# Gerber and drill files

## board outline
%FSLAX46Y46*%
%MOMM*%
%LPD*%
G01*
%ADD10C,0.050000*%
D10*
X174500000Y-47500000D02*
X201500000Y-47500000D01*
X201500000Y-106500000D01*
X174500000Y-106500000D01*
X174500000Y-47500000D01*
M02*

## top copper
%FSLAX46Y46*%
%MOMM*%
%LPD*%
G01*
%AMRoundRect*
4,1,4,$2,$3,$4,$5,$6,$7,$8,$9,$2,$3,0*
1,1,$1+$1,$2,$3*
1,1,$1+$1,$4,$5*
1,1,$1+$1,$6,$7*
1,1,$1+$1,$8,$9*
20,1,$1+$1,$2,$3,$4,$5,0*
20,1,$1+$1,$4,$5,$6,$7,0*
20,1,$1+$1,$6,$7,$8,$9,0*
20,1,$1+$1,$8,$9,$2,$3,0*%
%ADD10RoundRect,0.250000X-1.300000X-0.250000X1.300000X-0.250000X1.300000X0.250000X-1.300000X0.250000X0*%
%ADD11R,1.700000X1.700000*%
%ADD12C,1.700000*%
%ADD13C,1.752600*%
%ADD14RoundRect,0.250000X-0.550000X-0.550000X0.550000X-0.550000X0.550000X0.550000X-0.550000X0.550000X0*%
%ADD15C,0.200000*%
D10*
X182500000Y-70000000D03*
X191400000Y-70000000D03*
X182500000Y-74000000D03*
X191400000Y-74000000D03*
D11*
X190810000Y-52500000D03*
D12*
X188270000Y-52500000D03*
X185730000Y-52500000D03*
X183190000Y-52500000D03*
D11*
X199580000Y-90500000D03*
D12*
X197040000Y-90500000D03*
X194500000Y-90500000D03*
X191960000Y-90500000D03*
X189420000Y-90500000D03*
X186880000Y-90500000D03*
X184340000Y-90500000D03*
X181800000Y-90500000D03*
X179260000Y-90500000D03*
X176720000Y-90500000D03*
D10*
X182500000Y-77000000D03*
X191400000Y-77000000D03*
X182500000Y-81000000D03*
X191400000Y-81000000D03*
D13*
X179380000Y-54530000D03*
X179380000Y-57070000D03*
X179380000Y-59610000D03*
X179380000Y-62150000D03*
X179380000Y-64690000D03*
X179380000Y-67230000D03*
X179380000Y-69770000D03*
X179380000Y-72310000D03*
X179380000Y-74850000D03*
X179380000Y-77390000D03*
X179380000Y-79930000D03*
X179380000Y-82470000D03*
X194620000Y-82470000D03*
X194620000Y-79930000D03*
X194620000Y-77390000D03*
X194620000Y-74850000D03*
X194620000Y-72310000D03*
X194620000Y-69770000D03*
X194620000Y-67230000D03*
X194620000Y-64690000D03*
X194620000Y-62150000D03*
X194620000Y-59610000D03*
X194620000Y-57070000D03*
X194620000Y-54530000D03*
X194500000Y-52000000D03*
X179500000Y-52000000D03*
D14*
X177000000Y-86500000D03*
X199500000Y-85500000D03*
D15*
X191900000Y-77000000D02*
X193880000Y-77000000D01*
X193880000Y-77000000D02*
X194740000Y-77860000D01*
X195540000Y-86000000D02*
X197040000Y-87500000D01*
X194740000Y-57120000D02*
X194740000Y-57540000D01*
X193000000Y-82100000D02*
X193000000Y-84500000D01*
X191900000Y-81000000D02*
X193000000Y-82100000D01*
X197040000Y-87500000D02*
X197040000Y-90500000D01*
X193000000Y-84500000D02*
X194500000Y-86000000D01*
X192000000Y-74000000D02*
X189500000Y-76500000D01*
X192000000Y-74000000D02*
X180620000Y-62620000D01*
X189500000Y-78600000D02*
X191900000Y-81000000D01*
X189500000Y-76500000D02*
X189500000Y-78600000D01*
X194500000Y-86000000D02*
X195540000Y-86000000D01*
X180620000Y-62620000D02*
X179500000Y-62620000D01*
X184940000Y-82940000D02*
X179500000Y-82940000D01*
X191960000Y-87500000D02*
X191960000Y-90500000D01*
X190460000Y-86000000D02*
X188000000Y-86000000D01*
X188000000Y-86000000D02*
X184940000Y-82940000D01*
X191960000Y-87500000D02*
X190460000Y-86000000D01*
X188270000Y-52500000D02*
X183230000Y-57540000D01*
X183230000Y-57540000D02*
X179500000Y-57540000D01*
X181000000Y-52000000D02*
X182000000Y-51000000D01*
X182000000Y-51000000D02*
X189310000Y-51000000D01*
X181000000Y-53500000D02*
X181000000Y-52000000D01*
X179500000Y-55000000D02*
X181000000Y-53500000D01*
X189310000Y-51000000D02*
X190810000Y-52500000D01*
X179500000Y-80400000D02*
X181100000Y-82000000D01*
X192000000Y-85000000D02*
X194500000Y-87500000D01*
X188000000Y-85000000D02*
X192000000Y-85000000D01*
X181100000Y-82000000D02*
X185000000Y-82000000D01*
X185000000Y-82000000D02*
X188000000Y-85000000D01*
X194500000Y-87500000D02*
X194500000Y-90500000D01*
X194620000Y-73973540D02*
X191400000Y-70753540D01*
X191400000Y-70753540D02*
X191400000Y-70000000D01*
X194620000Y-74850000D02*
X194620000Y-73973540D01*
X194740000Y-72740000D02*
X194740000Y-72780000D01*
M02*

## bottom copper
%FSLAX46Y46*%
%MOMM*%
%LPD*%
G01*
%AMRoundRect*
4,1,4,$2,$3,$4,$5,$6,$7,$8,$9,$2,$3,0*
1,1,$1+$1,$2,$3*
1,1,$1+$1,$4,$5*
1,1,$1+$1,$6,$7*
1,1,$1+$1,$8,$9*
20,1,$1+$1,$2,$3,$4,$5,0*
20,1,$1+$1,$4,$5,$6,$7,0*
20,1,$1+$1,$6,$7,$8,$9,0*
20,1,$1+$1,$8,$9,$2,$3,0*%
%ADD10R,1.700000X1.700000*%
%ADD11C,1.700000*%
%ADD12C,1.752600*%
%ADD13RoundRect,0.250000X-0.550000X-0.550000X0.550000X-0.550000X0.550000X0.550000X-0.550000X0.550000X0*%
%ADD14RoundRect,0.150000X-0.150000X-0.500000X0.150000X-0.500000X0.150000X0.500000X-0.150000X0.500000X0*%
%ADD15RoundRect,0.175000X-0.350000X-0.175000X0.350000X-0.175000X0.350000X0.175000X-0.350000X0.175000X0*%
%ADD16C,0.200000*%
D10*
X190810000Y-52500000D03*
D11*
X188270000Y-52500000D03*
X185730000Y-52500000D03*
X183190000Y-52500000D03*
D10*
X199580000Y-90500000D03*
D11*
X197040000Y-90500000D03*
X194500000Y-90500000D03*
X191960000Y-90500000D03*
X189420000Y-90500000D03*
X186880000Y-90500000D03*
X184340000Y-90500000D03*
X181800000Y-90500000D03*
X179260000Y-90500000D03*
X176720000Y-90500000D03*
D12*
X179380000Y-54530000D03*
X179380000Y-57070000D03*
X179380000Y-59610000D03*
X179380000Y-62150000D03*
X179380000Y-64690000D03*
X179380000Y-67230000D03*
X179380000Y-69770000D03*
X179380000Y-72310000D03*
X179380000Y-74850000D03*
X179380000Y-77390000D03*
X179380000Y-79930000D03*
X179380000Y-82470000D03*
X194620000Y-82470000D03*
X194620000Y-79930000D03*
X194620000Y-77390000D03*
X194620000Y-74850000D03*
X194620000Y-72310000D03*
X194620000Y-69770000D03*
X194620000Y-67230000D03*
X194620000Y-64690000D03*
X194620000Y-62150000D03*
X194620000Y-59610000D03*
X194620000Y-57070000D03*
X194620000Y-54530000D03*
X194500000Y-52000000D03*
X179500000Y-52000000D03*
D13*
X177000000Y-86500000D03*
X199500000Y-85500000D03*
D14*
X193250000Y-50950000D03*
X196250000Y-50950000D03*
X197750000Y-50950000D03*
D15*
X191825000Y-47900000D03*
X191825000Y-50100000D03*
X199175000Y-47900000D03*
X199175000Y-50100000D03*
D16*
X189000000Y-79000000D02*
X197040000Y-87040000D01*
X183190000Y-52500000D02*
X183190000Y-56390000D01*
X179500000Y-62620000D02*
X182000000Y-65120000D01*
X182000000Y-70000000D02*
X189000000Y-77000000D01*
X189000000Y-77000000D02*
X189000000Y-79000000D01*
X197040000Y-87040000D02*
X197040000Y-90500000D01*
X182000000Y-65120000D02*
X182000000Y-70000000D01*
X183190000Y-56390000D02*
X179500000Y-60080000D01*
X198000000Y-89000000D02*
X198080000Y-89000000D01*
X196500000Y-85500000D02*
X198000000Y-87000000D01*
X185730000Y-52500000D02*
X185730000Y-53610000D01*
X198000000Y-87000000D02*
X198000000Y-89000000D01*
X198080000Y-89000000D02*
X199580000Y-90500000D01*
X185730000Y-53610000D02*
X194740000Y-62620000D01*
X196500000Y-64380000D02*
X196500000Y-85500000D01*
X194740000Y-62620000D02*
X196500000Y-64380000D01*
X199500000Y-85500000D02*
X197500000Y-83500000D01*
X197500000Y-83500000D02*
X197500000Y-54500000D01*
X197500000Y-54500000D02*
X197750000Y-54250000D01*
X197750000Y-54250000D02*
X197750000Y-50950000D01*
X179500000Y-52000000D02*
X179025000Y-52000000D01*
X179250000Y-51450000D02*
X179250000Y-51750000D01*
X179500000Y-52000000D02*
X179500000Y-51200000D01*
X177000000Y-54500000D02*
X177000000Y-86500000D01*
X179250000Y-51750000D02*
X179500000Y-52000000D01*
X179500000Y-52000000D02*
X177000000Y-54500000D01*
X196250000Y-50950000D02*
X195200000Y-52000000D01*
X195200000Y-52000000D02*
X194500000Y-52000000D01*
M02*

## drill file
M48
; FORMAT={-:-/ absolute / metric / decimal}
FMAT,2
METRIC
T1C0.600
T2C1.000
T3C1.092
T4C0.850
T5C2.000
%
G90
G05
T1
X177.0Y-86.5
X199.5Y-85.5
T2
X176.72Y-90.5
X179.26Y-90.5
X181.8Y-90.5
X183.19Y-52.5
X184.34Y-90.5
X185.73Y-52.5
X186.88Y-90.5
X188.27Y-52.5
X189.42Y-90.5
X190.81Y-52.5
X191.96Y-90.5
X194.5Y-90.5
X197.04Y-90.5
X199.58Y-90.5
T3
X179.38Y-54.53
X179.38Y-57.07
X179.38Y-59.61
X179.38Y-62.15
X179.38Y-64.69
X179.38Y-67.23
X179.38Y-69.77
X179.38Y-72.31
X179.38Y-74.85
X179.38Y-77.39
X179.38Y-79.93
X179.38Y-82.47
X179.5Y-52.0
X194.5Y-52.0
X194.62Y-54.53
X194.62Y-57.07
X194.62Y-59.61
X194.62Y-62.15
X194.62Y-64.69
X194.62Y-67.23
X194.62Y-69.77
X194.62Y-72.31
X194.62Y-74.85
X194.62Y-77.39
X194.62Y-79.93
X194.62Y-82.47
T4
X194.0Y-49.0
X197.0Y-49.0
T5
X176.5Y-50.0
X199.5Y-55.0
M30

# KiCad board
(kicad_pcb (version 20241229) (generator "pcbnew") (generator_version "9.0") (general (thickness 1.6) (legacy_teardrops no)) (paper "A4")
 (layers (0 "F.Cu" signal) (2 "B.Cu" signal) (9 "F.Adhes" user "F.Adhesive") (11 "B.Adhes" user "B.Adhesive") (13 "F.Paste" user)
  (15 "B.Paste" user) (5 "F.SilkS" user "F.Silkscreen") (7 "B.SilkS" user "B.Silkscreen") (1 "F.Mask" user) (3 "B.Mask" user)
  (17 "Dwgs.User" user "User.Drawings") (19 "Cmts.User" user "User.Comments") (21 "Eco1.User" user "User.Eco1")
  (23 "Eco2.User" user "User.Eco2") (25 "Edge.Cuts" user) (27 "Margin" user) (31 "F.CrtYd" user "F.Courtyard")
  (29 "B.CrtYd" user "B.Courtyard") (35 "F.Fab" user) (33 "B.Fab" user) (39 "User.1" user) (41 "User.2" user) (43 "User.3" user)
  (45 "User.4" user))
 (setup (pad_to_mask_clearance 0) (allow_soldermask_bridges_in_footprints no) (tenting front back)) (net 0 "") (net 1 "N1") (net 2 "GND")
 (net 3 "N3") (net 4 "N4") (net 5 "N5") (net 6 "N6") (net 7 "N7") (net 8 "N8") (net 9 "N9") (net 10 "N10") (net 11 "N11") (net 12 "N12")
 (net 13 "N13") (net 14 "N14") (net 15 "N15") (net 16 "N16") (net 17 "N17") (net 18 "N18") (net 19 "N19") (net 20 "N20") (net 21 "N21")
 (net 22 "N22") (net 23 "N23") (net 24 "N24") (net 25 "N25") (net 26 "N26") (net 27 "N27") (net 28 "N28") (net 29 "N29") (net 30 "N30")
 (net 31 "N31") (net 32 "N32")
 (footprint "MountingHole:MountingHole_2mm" (layer "F.Cu") (at 176.5 50)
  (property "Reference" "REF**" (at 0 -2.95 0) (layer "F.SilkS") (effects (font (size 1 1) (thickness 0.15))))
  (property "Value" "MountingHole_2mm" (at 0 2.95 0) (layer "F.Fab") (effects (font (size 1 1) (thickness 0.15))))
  (pad "" np_thru_hole circle (at 0 0) (size 2 2) (drill 2) (layers "*.Cu" "*.Mask")))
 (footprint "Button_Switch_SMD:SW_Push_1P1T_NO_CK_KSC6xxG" (layer "F.Cu") (at 186.95 72)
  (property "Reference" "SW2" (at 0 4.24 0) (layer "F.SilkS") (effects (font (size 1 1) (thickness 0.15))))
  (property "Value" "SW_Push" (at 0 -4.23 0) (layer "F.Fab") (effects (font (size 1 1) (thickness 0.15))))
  (pad "1" smd roundrect (at -4.45 -2) (size 3.1 1) (layers "F.Cu" "F.Mask" "F.Paste") (roundrect_rratio 0.25) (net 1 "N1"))
  (pad "1" smd roundrect (at 4.45 -2) (size 3.1 1) (layers "F.Cu" "F.Mask" "F.Paste") (roundrect_rratio 0.25) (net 1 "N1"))
  (pad "2" smd roundrect (at -4.45 2) (size 3.1 1) (layers "F.Cu" "F.Mask" "F.Paste") (roundrect_rratio 0.25) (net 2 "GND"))
  (pad "2" smd roundrect (at 4.45 2) (size 3.1 1) (layers "F.Cu" "F.Mask" "F.Paste") (roundrect_rratio 0.25) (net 2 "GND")))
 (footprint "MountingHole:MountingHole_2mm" (layer "F.Cu") (at 199.5 55)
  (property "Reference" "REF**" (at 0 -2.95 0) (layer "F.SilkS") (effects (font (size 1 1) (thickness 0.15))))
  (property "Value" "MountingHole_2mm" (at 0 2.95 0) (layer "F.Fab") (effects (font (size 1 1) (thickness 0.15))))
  (pad "" np_thru_hole circle (at 0 0) (size 2 2) (drill 2) (layers "*.Cu" "*.Mask")))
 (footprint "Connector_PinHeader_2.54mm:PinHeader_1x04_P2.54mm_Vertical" (layer "F.Cu") (at 190.81 52.5 -90)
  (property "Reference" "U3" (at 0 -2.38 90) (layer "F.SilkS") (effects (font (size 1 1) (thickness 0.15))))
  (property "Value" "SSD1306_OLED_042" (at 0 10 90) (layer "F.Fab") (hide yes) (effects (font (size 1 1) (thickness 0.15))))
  (pad "1" thru_hole rect (at 0 0 270) (size 1.7 1.7) (drill 1) (layers "*.Cu" "*.Mask") (remove_unused_layers no) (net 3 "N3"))
  (pad "2" thru_hole circle (at 0 2.54 270) (size 1.7 1.7) (drill 1) (layers "*.Cu" "*.Mask") (remove_unused_layers no) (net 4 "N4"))
  (pad "3" thru_hole circle (at 0 5.08 270) (size 1.7 1.7) (drill 1) (layers "*.Cu" "*.Mask") (remove_unused_layers no) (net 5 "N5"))
  (pad "4" thru_hole circle (at 0 7.62 270) (size 1.7 1.7) (drill 1) (layers "*.Cu" "*.Mask") (remove_unused_layers no) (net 2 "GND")))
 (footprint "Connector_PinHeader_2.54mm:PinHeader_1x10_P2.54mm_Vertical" (layer "F.Cu") (at 199.58 90.5 -90)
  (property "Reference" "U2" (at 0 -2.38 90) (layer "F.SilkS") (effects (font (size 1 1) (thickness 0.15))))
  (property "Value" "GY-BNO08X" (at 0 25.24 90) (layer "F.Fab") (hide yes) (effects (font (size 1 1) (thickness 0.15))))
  (pad "1" thru_hole rect (at 0 0 270) (size 1.7 1.7) (drill 1) (layers "*.Cu" "*.Mask") (remove_unused_layers no) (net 5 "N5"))
  (pad "2" thru_hole circle (at 0 2.54 270) (size 1.7 1.7) (drill 1) (layers "*.Cu" "*.Mask") (remove_unused_layers no) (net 2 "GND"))
  (pad "3" thru_hole circle (at 0 5.08 270) (size 1.7 1.7) (drill 1) (layers "*.Cu" "*.Mask") (remove_unused_layers no) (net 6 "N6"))
  (pad "4" thru_hole circle (at 0 7.62 270) (size 1.7 1.7) (drill 1) (layers "*.Cu" "*.Mask") (remove_unused_layers no) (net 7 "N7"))
  (pad "5" thru_hole circle (at 0 10.16 270) (size 1.7 1.7) (drill 1) (layers "*.Cu" "*.Mask") (remove_unused_layers no) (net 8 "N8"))
  (pad "6" thru_hole circle (at 0 12.7 270) (size 1.7 1.7) (drill 1) (layers "*.Cu" "*.Mask") (remove_unused_layers no) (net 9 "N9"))
  (pad "7" thru_hole circle (at 0 15.24 270) (size 1.7 1.7) (drill 1) (layers "*.Cu" "*.Mask") (remove_unused_layers no) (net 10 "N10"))
  (pad "8" thru_hole circle (at 0 17.78 270) (size 1.7 1.7) (drill 1) (layers "*.Cu" "*.Mask") (remove_unused_layers no) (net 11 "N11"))
  (pad "9" thru_hole circle (at 0 20.32 270) (size 1.7 1.7) (drill 1) (layers "*.Cu" "*.Mask") (remove_unused_layers no) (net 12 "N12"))
  (pad "10" thru_hole circle (at 0 22.86 270) (size 1.7 1.7) (drill 1) (layers "*.Cu" "*.Mask") (remove_unused_layers no) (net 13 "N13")))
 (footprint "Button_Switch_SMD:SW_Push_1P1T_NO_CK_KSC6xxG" (layer "F.Cu") (at 186.95 79)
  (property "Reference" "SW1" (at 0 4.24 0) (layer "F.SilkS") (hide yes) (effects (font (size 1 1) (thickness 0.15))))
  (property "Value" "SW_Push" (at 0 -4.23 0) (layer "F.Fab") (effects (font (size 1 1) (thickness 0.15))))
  (pad "1" smd roundrect (at -4.45 -2) (size 3.1 1) (layers "F.Cu" "F.Mask" "F.Paste") (roundrect_rratio 0.25) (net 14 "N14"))
  (pad "1" smd roundrect (at 4.45 -2) (size 3.1 1) (layers "F.Cu" "F.Mask" "F.Paste") (roundrect_rratio 0.25) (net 14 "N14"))
  (pad "2" smd roundrect (at -4.45 2) (size 3.1 1) (layers "F.Cu" "F.Mask" "F.Paste") (roundrect_rratio 0.25) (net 2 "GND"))
  (pad "2" smd roundrect (at 4.45 2) (size 3.1 1) (layers "F.Cu" "F.Mask" "F.Paste") (roundrect_rratio 0.25) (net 2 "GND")))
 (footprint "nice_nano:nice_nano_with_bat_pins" (layer "F.Cu") (at 187 68.5 -90)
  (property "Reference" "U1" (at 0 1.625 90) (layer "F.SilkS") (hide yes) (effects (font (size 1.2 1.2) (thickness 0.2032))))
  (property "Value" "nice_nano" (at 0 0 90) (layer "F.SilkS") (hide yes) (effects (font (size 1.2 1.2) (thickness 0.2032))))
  (pad "1" thru_hole circle (at -13.97 7.62 270) (size 1.7526 1.7526) (drill 1.0922) (layers "*.Cu" "*.SilkS" "*.Mask")
   (remove_unused_layers no) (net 3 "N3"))
  (pad "2" thru_hole circle (at -11.43 7.62 270) (size 1.7526 1.7526) (drill 1.0922) (layers "*.Cu" "*.SilkS" "*.Mask")
   (remove_unused_layers no) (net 4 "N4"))
  (pad "3" thru_hole circle (at -8.89 7.62 270) (size 1.7526 1.7526) (drill 1.0922) (layers "*.Cu" "*.SilkS" "*.Mask")
   (remove_unused_layers no) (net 2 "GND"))
  (pad "4" thru_hole circle (at -6.35 7.62 270) (size 1.7526 1.7526) (drill 1.0922) (layers "*.Cu" "*.SilkS" "*.Mask")
   (remove_unused_layers no) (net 2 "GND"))
  (pad "5" thru_hole circle (at -3.81 7.62 270) (size 1.7526 1.7526) (drill 1.0922) (layers "*.Cu" "*.SilkS" "*.Mask")
   (remove_unused_layers no) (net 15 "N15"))
  (pad "6" thru_hole circle (at -1.27 7.62 270) (size 1.7526 1.7526) (drill 1.0922) (layers "*.Cu" "*.SilkS" "*.Mask")
   (remove_unused_layers no) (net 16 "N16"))
  (pad "7" thru_hole circle (at 1.27 7.62 270) (size 1.7526 1.7526) (drill 1.0922) (layers "*.Cu" "*.SilkS" "*.Mask")
   (remove_unused_layers no) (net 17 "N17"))
  (pad "8" thru_hole circle (at 3.81 7.62 270) (size 1.7526 1.7526) (drill 1.0922) (layers "*.Cu" "*.SilkS" "*.Mask")
   (remove_unused_layers no) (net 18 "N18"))
  (pad "9" thru_hole circle (at 6.35 7.62 270) (size 1.7526 1.7526) (drill 1.0922) (layers "*.Cu" "*.SilkS" "*.Mask")
   (remove_unused_layers no) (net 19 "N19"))
  (pad "10" thru_hole circle (at 8.89 7.62 270) (size 1.7526 1.7526) (drill 1.0922) (layers "*.Cu" "*.SilkS" "*.Mask")
   (remove_unused_layers no) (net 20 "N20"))
  (pad "11" thru_hole circle (at 11.43 7.62 270) (size 1.7526 1.7526) (drill 1.0922) (layers "*.Cu" "*.SilkS" "*.Mask")
   (remove_unused_layers no) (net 6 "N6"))
  (pad "12" thru_hole circle (at 13.97 7.62 270) (size 1.7526 1.7526) (drill 1.0922) (layers "*.Cu" "*.SilkS" "*.Mask")
   (remove_unused_layers no) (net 7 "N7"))
  (pad "13" thru_hole circle (at 13.97 -7.62 270) (size 1.7526 1.7526) (drill 1.0922) (layers "*.Cu" "*.SilkS" "*.Mask")
   (remove_unused_layers no) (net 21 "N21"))
  (pad "14" thru_hole circle (at 11.43 -7.62 270) (size 1.7526 1.7526) (drill 1.0922) (layers "*.Cu" "*.SilkS" "*.Mask")
   (remove_unused_layers no) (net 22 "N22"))
  (pad "15" thru_hole circle (at 8.89 -7.62 270) (size 1.7526 1.7526) (drill 1.0922) (layers "*.Cu" "*.SilkS" "*.Mask")
   (remove_unused_layers no) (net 14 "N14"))
  (pad "16" thru_hole circle (at 6.35 -7.62 270) (size 1.7526 1.7526) (drill 1.0922) (layers "*.Cu" "*.SilkS" "*.Mask")
   (remove_unused_layers no) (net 1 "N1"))
  (pad "17" thru_hole circle (at 3.81 -7.62 270) (size 1.7526 1.7526) (drill 1.0922) (layers "*.Cu" "*.SilkS" "*.Mask")
   (remove_unused_layers no) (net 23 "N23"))
  (pad "18" thru_hole circle (at 1.27 -7.62 270) (size 1.7526 1.7526) (drill 1.0922) (layers "*.Cu" "*.SilkS" "*.Mask")
   (remove_unused_layers no) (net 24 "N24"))
  (pad "19" thru_hole circle (at -1.27 -7.62 270) (size 1.7526 1.7526) (drill 1.0922) (layers "*.Cu" "*.SilkS" "*.Mask")
   (remove_unused_layers no) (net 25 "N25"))
  (pad "20" thru_hole circle (at -3.81 -7.62 270) (size 1.7526 1.7526) (drill 1.0922) (layers "*.Cu" "*.SilkS" "*.Mask")
   (remove_unused_layers no) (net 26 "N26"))
  (pad "21" thru_hole circle (at -6.35 -7.62 270) (size 1.7526 1.7526) (drill 1.0922) (layers "*.Cu" "*.SilkS" "*.Mask")
   (remove_unused_layers no) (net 5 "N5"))
  (pad "22" thru_hole circle (at -8.89 -7.62 270) (size 1.7526 1.7526) (drill 1.0922) (layers "*.Cu" "*.SilkS" "*.Mask")
   (remove_unused_layers no) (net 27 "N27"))
  (pad "23" thru_hole circle (at -11.43 -7.62 270) (size 1.7526 1.7526) (drill 1.0922) (layers "*.Cu" "*.SilkS" "*.Mask")
   (remove_unused_layers no) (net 2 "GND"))
  (pad "24" thru_hole circle (at -13.97 -7.62 270) (size 1.7526 1.7526) (drill 1.0922) (layers "*.Cu" "*.SilkS" "*.Mask")
   (remove_unused_layers no) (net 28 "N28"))
  (pad "25" thru_hole circle (at -16.5 -7.5 270) (size 1.7526 1.7526) (drill 1.0922) (layers "*.Cu" "*.SilkS" "*.Mask")
   (remove_unused_layers no) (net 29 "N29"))
  (pad "26" thru_hole circle (at -16.5 7.5 270) (size 1.7526 1.7526) (drill 1.0922) (layers "*.Cu" "*.SilkS" "*.Mask")
   (remove_unused_layers no) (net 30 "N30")))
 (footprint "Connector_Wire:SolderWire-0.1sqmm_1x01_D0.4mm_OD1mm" (layer "B.Cu") (at 177 86.5)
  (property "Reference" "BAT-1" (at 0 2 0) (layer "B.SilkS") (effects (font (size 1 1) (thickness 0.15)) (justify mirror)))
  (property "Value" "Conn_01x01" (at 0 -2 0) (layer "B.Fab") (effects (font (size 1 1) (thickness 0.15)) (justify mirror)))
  (pad "1" thru_hole roundrect (at 0 0) (size 1.6 1.6) (drill 0.6) (layers "*.Cu" "*.Mask") (remove_unused_layers no)
   (roundrect_rratio 0.15625) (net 30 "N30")))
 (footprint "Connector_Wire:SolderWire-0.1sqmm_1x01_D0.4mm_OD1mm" (layer "B.Cu") (at 199.5 85.5)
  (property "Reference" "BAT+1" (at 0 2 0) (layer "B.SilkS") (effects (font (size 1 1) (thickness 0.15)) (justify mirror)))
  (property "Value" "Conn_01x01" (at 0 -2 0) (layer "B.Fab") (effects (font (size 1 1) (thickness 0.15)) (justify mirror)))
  (pad "1" thru_hole roundrect (at 0 0) (size 1.6 1.6) (drill 0.6) (layers "*.Cu" "*.Mask") (remove_unused_layers no)
   (roundrect_rratio 0.15625) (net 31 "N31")))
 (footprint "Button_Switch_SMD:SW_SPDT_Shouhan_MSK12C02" (layer "B.Cu") (at 195.5 49)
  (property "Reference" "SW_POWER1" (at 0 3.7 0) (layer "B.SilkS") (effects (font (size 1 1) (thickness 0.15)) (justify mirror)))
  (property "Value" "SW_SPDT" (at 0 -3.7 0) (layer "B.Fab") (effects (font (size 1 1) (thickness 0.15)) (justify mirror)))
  (pad "" np_thru_hole circle (at -1.5 0) (size 0.85 0.85) (drill 0.85) (layers "*.Mask"))
  (pad "" np_thru_hole circle (at 1.5 0) (size 0.85 0.85) (drill 0.85) (layers "*.Mask"))
  (pad "1" smd roundrect (at -2.25 1.95) (size 0.6 1.3) (layers "B.Cu" "B.Mask" "B.Paste") (roundrect_rratio 0.25) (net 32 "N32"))
  (pad "2" smd roundrect (at 0.75 1.95) (size 0.6 1.3) (layers "B.Cu" "B.Mask" "B.Paste") (roundrect_rratio 0.25) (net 29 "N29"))
  (pad "3" smd roundrect (at 2.25 1.95) (size 0.6 1.3) (layers "B.Cu" "B.Mask" "B.Paste") (roundrect_rratio 0.25) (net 31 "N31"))
  (pad "SH" smd roundrect (at -3.675 -1.1) (size 1.05 0.7) (layers "B.Cu" "B.Mask" "B.Paste") (roundrect_rratio 0.25))
  (pad "SH" smd roundrect (at -3.675 1.1) (size 1.05 0.7) (layers "B.Cu" "B.Mask" "B.Paste") (roundrect_rratio 0.25))
  (pad "SH" smd roundrect (at 3.675 -1.1) (size 1.05 0.7) (layers "B.Cu" "B.Mask" "B.Paste") (roundrect_rratio 0.25))
  (pad "SH" smd roundrect (at 3.675 1.1) (size 1.05 0.7) (layers "B.Cu" "B.Mask" "B.Paste") (roundrect_rratio 0.25)))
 (gr_rect (start 174.5 47.5) (end 201.5 106.5) (stroke (width 0.05) (type default)) (fill no) (layer "Edge.Cuts"))
 (segment (start 191.9 77) (end 193.88 77) (width 0.2) (layer "F.Cu") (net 14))
 (segment (start 193.88 77) (end 194.74 77.86) (width 0.2) (layer "F.Cu") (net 14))
 (segment (start 195.54 86) (end 197.04 87.5) (width 0.2) (layer "F.Cu") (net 2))
 (segment (start 194.74 57.12) (end 194.74 57.54) (width 0.2) (layer "F.Cu") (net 2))
 (segment (start 193 82.1) (end 193 84.5) (width 0.2) (layer "F.Cu") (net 2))
 (segment (start 191.9 81) (end 193 82.1) (width 0.2) (layer "F.Cu") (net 2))
 (segment (start 197.04 87.5) (end 197.04 90.5) (width 0.2) (layer "F.Cu") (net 2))
 (segment (start 193 84.5) (end 194.5 86) (width 0.2) (layer "F.Cu") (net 2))
 (segment (start 192 74) (end 189.5 76.5) (width 0.2) (layer "F.Cu") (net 2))
 (segment (start 192 74) (end 180.62 62.62) (width 0.2) (layer "F.Cu") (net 2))
 (segment (start 189.5 78.6) (end 191.9 81) (width 0.2) (layer "F.Cu") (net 2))
 (segment (start 189.5 76.5) (end 189.5 78.6) (width 0.2) (layer "F.Cu") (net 2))
 (segment (start 194.5 86) (end 195.54 86) (width 0.2) (layer "F.Cu") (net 2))
 (segment (start 180.62 62.62) (end 179.5 62.62) (width 0.2) (layer "F.Cu") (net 2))
 (segment (start 189 79) (end 197.04 87.04) (width 0.2) (layer "B.Cu") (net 2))
 (segment (start 183.19 52.5) (end 183.19 56.39) (width 0.2) (layer "B.Cu") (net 2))
 (segment (start 179.5 62.62) (end 182 65.12) (width 0.2) (layer "B.Cu") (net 2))
 (segment (start 182 70) (end 189 77) (width 0.2) (layer "B.Cu") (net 2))
 (segment (start 189 77) (end 189 79) (width 0.2) (layer "B.Cu") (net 2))
 (segment (start 197.04 87.04) (end 197.04 90.5) (width 0.2) (layer "B.Cu") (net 2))
 (segment (start 182 65.12) (end 182 70) (width 0.2) (layer "B.Cu") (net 2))
 (segment (start 183.19 56.39) (end 179.5 60.08) (width 0.2) (layer "B.Cu") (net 2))
 (segment (start 184.94 82.94) (end 179.5 82.94) (width 0.2) (layer "F.Cu") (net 7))
 (segment (start 191.96 87.5) (end 191.96 90.5) (width 0.2) (layer "F.Cu") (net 7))
 (segment (start 190.46 86) (end 188 86) (width 0.2) (layer "F.Cu") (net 7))
 (segment (start 188 86) (end 184.94 82.94) (width 0.2) (layer "F.Cu") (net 7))
 (segment (start 191.96 87.5) (end 190.46 86) (width 0.2) (layer "F.Cu") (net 7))
 (segment (start 188.27 52.5) (end 183.23 57.54) (width 0.2) (layer "F.Cu") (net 4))
 (segment (start 183.23 57.54) (end 179.5 57.54) (width 0.2) (layer "F.Cu") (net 4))
 (segment (start 198 89) (end 198.08 89) (width 0.2) (layer "B.Cu") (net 5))
 (segment (start 196.5 85.5) (end 198 87) (width 0.2) (layer "B.Cu") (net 5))
 (segment (start 185.73 52.5) (end 185.73 53.61) (width 0.2) (layer "B.Cu") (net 5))
 (segment (start 198 87) (end 198 89) (width 0.2) (layer "B.Cu") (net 5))
 (segment (start 198.08 89) (end 199.58 90.5) (width 0.2) (layer "B.Cu") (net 5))
 (segment (start 185.73 53.61) (end 194.74 62.62) (width 0.2) (layer "B.Cu") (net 5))
 (segment (start 196.5 64.38) (end 196.5 85.5) (width 0.2) (layer "B.Cu") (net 5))
 (segment (start 194.74 62.62) (end 196.5 64.38) (width 0.2) (layer "B.Cu") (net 5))
 (segment (start 181 52) (end 182 51) (width 0.2) (layer "F.Cu") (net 3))
 (segment (start 182 51) (end 189.31 51) (width 0.2) (layer "F.Cu") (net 3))
 (segment (start 181 53.5) (end 181 52) (width 0.2) (layer "F.Cu") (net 3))
 (segment (start 179.5 55) (end 181 53.5) (width 0.2) (layer "F.Cu") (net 3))
 (segment (start 189.31 51) (end 190.81 52.5) (width 0.2) (layer "F.Cu") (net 3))
 (segment (start 179.5 80.4) (end 181.1 82) (width 0.2) (layer "F.Cu") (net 6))
 (segment (start 192 85) (end 194.5 87.5) (width 0.2) (layer "F.Cu") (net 6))
 (segment (start 188 85) (end 192 85) (width 0.2) (layer "F.Cu") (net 6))
 (segment (start 181.1 82) (end 185 82) (width 0.2) (layer "F.Cu") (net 6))
 (segment (start 185 82) (end 188 85) (width 0.2) (layer "F.Cu") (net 6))
 (segment (start 194.5 87.5) (end 194.5 90.5) (width 0.2) (layer "F.Cu") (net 6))
 (segment (start 194.62 73.97354) (end 191.4 70.75354) (width 0.2) (layer "F.Cu") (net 1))
 (segment (start 191.4 70.75354) (end 191.4 70) (width 0.2) (layer "F.Cu") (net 1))
 (segment (start 194.62 74.85) (end 194.62 73.97354) (width 0.2) (layer "F.Cu") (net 1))
 (segment (start 194.74 72.74) (end 194.74 72.78) (width 0.2) (layer "F.Cu") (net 23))
 (segment (start 199.5 85.5) (end 197.5 83.5) (width 0.2) (layer "B.Cu") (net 31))
 (segment (start 197.5 83.5) (end 197.5 54.5) (width 0.2) (layer "B.Cu") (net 31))
 (segment (start 197.5 54.5) (end 197.75 54.25) (width 0.2) (layer "B.Cu") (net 31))
 (segment (start 197.75 54.25) (end 197.75 50.95) (width 0.2) (layer "B.Cu") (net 31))
 (segment (start 179.5 52) (end 179.025 52) (width 0.2) (layer "B.Cu") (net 30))
 (segment (start 179.25 51.45) (end 179.25 51.75) (width 0.2) (layer "B.Cu") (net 30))
 (segment (start 179.5 52) (end 179.5 51.2) (width 0.2) (layer "B.Cu") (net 30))
 (segment (start 177 54.5) (end 177 86.5) (width 0.2) (layer "B.Cu") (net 30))
 (segment (start 179.25 51.75) (end 179.5 52) (width 0.2) (layer "B.Cu") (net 30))
 (segment (start 179.5 52) (end 177 54.5) (width 0.2) (layer "B.Cu") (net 30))
 (segment (start 196.25 50.95) (end 195.2 52) (width 0.2) (layer "B.Cu") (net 29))
 (segment (start 195.2 52) (end 194.5 52) (width 0.2) (layer "B.Cu") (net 29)))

